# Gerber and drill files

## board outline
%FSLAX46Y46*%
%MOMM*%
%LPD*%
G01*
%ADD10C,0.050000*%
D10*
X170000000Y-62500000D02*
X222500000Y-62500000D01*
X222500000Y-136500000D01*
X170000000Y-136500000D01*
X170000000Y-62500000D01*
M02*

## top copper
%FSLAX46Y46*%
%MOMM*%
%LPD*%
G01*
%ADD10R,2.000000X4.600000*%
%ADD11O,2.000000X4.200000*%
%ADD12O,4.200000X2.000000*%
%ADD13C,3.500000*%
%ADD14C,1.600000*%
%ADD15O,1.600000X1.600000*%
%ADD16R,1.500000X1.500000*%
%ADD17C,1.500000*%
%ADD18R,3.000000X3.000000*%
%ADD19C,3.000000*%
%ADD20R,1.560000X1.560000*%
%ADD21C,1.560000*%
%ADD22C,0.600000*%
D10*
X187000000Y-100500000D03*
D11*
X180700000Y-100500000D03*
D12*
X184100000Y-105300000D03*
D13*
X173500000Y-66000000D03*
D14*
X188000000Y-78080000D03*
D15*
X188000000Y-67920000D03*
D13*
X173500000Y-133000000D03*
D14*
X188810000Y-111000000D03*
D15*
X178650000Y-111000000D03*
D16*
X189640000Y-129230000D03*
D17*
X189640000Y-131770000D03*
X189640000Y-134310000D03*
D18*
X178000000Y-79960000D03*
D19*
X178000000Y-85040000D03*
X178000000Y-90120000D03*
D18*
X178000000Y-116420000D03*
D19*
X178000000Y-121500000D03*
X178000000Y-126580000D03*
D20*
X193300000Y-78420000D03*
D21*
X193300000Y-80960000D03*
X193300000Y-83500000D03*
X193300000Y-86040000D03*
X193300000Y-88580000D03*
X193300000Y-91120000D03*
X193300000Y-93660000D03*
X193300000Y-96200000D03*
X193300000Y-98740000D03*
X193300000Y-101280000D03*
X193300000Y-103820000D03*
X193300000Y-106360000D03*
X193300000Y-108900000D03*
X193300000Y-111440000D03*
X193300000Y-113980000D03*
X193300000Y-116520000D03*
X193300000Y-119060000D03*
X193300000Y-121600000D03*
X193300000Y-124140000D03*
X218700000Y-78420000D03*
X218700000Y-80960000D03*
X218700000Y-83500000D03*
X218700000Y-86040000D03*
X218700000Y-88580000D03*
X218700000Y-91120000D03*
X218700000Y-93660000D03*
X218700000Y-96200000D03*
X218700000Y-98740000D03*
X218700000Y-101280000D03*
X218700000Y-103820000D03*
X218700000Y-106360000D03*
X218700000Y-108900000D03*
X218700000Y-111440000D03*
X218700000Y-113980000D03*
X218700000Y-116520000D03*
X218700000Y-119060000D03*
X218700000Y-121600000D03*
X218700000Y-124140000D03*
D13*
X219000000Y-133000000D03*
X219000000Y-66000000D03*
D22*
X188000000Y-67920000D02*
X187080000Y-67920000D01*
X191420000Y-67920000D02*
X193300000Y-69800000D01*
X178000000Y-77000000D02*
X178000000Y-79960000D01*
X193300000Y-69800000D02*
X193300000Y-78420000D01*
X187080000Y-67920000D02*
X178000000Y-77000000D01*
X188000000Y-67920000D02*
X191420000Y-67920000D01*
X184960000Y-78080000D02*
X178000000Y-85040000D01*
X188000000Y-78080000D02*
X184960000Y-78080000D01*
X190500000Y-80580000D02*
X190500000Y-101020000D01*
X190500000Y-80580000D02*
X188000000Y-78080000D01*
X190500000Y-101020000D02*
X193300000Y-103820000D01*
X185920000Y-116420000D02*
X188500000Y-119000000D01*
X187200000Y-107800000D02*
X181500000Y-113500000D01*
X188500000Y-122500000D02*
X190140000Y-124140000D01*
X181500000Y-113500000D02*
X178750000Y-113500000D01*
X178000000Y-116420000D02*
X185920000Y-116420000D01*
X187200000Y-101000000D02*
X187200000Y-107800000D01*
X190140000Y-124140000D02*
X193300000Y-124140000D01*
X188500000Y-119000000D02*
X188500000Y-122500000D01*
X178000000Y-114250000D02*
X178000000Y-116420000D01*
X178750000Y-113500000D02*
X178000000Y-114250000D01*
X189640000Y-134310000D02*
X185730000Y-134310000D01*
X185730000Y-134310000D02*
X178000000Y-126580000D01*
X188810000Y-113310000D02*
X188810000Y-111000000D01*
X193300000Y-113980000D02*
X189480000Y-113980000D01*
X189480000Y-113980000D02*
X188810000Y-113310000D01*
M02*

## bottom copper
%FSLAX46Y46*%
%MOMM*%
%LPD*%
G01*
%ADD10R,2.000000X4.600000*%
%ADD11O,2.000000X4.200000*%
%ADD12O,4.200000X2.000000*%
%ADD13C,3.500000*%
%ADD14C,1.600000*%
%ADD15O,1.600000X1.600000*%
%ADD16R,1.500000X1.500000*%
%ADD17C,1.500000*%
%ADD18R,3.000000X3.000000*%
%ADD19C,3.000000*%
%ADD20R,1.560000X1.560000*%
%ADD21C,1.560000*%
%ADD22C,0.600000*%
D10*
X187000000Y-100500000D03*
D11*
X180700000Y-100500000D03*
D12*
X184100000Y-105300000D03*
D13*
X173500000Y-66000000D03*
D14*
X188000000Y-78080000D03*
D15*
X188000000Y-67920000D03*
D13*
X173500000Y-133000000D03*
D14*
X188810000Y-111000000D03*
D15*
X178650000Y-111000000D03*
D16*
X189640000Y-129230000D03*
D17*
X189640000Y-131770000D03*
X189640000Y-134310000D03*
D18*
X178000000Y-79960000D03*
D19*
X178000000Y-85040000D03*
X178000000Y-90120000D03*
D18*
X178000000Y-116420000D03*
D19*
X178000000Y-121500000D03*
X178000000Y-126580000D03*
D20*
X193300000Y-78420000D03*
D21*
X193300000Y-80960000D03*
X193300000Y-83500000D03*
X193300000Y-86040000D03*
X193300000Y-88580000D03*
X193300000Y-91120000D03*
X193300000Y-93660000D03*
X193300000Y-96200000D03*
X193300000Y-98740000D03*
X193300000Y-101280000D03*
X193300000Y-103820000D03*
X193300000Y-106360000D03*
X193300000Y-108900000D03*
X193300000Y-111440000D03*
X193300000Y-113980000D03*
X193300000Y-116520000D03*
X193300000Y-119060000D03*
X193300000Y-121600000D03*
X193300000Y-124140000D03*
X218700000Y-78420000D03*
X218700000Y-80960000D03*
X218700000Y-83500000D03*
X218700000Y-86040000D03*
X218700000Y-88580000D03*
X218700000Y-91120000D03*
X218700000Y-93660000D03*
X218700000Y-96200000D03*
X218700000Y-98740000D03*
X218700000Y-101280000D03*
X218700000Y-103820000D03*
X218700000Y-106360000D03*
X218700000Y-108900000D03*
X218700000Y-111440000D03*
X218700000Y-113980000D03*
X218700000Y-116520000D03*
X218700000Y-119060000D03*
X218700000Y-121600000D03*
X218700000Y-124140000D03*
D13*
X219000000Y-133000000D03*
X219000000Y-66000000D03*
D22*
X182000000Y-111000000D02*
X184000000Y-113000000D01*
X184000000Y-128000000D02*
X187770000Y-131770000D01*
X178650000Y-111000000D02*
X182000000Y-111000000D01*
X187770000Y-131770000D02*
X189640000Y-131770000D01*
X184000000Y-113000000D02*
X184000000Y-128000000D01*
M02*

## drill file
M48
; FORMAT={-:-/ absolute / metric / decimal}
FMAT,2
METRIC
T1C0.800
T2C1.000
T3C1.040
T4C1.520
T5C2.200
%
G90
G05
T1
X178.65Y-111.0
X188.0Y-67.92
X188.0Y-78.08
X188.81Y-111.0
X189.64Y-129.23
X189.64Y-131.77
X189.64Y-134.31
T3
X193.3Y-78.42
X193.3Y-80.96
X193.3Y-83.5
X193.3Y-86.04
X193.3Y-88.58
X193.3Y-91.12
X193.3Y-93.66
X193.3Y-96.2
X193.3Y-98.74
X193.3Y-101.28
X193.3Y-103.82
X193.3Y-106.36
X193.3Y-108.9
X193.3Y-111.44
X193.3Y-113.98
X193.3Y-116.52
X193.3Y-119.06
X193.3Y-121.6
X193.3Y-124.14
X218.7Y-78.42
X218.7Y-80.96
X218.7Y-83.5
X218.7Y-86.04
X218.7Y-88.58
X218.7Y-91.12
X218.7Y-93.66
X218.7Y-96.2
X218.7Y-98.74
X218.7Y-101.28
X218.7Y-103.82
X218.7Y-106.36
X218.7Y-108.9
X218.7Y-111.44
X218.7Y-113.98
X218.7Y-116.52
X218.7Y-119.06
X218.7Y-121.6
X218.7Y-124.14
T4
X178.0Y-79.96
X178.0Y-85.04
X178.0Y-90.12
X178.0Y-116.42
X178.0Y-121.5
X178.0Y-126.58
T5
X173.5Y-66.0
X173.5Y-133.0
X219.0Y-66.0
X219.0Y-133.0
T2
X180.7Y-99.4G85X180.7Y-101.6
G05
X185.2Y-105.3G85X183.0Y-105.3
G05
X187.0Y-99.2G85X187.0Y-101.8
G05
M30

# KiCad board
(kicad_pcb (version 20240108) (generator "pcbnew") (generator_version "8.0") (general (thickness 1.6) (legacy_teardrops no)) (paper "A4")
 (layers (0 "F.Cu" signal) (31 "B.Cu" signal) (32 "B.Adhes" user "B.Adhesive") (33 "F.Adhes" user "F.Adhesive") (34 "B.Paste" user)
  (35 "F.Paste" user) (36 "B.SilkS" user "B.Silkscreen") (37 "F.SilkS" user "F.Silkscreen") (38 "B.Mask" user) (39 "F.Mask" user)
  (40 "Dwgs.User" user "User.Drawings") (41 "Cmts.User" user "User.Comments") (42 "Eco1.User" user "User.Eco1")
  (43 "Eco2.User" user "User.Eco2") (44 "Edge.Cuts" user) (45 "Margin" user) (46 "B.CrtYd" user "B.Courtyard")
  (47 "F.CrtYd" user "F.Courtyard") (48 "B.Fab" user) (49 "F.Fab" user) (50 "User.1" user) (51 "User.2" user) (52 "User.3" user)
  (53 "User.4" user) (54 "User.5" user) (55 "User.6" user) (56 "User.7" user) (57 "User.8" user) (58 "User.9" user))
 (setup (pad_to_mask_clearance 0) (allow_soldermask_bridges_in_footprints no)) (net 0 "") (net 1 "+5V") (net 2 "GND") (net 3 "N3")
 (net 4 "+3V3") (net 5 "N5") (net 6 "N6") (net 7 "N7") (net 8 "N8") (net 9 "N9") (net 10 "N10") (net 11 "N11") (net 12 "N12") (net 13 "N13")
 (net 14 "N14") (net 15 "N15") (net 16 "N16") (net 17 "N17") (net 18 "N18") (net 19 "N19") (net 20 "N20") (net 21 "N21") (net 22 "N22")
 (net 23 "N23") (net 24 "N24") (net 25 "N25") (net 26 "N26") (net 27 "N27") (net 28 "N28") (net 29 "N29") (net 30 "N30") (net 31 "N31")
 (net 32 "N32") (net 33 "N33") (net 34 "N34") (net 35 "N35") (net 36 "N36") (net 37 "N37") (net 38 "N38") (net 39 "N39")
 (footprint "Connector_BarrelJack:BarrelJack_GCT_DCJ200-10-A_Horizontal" (layer "F.Cu") (at 187 100.5 -90)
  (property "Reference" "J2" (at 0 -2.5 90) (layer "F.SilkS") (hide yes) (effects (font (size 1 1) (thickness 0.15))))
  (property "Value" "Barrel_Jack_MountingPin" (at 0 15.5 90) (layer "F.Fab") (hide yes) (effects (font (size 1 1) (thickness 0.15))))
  (pad "1" thru_hole rect (at 0 0 270) (size 4.6 2) (drill oval 3.6 1) (layers "*.Cu" "*.Mask") (remove_unused_layers no) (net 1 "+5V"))
  (pad "2" thru_hole oval (at 0 6.3 270) (size 4.2 2) (drill oval 3.2 1) (layers "*.Cu" "*.Mask") (remove_unused_layers no) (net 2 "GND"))
  (pad "3" thru_hole oval (at 4.8 2.9 270) (size 2 4.2) (drill oval 1 3.2) (layers "*.Cu" "*.Mask") (remove_unused_layers no)))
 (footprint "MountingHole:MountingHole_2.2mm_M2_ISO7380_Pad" (layer "F.Cu") (at 173.5 66)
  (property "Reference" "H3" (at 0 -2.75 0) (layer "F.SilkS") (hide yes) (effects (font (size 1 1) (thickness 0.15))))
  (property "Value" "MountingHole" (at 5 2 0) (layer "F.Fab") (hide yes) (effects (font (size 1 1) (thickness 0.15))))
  (pad "1" thru_hole circle (at 0 0) (size 3.5 3.5) (drill 2.2) (layers "*.Cu" "*.Mask") (remove_unused_layers no)))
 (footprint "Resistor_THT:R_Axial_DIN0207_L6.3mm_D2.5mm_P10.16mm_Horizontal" (layer "F.Cu") (at 188 78.08 90)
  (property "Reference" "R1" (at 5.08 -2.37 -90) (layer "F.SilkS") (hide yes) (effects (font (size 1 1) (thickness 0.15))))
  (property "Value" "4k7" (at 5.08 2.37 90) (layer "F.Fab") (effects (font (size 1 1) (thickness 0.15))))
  (pad "1" thru_hole circle (at 0 0 90) (size 1.6 1.6) (drill 0.8) (layers "*.Cu" "*.Mask") (remove_unused_layers no) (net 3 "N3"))
  (pad "2" thru_hole oval (at 10.16 0 90) (size 1.6 1.6) (drill 0.8) (layers "*.Cu" "*.Mask") (remove_unused_layers no) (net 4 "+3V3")))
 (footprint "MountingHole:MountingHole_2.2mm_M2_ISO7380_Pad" (layer "F.Cu") (at 173.5 133)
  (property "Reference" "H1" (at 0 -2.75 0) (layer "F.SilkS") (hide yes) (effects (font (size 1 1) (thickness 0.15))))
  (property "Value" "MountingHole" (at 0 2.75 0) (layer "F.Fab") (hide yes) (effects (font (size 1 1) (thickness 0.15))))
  (pad "1" thru_hole circle (at 0 0) (size 3.5 3.5) (drill 2.2) (layers "*.Cu" "*.Mask") (remove_unused_layers no)))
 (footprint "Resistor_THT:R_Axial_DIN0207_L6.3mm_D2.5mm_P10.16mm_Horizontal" (layer "F.Cu") (at 188.81 111 180)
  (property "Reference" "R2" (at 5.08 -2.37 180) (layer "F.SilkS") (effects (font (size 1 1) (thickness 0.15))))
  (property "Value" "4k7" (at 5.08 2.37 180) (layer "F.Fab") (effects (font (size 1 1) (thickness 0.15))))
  (pad "1" thru_hole circle (at 0 0 180) (size 1.6 1.6) (drill 0.8) (layers "*.Cu" "*.Mask") (remove_unused_layers no) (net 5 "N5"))
  (pad "2" thru_hole oval (at 10.16 0 180) (size 1.6 1.6) (drill 0.8) (layers "*.Cu" "*.Mask") (remove_unused_layers no) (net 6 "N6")))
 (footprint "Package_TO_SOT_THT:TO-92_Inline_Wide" (layer "F.Cu") (at 189.64 129.23 -90)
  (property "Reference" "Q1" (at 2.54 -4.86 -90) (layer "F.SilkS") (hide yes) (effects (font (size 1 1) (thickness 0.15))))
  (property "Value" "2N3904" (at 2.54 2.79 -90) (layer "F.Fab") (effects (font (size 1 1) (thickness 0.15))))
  (pad "1" thru_hole rect (at 0 0 270) (size 1.5 1.5) (drill 0.8) (layers "*.Cu" "*.Mask") (remove_unused_layers no) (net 2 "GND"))
  (pad "2" thru_hole circle (at 2.54 0 270) (size 1.5 1.5) (drill 0.8) (layers "*.Cu" "*.Mask") (remove_unused_layers no) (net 6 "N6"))
  (pad "3" thru_hole circle (at 5.08 0 270) (size 1.5 1.5) (drill 0.8) (layers "*.Cu" "*.Mask") (remove_unused_layers no) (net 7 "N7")))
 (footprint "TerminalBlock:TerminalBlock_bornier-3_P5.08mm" (layer "F.Cu") (at 178 79.96 -90)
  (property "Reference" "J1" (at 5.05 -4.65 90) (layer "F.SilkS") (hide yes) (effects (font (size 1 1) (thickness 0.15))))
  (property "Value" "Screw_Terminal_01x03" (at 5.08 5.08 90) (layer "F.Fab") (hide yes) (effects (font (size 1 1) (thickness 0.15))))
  (pad "1" thru_hole rect (at 0 0 270) (size 3 3) (drill 1.52) (layers "*.Cu" "*.Mask") (remove_unused_layers no) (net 4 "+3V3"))
  (pad "2" thru_hole circle (at 5.08 0 270) (size 3 3) (drill 1.52) (layers "*.Cu" "*.Mask") (remove_unused_layers no) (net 3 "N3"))
  (pad "3" thru_hole circle (at 10.16 0 270) (size 3 3) (drill 1.52) (layers "*.Cu" "*.Mask") (remove_unused_layers no) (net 2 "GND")))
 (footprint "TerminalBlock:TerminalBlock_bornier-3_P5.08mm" (layer "F.Cu") (at 178 116.42 -90)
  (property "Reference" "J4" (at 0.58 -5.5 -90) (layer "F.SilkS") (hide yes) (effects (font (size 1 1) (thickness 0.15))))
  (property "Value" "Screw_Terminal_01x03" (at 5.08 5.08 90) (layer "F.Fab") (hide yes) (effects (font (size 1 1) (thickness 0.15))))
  (pad "1" thru_hole rect (at 0 0 270) (size 3 3) (drill 1.52) (layers "*.Cu" "*.Mask") (remove_unused_layers no) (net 1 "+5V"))
  (pad "2" thru_hole circle (at 5.08 0 270) (size 3 3) (drill 1.52) (layers "*.Cu" "*.Mask") (remove_unused_layers no) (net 2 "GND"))
  (pad "3" thru_hole circle (at 10.16 0 270) (size 3 3) (drill 1.52) (layers "*.Cu" "*.Mask") (remove_unused_layers no) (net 7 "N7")))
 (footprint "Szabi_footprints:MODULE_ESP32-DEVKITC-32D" (layer "F.Cu") (at 206 98.18)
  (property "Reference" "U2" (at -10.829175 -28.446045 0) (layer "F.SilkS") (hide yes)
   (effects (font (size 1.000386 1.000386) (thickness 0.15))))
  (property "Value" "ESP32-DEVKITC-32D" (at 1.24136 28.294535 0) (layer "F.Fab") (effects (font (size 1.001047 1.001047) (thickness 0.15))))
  (pad "J2-1" thru_hole rect (at -12.7 -19.76) (size 1.56 1.56) (drill 1.04) (layers "*.Cu" "*.Mask") (remove_unused_layers no)
   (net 4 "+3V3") (solder_mask_margin 0.102))
  (pad "J2-2" thru_hole circle (at -12.7 -17.22) (size 1.56 1.56) (drill 1.04) (layers "*.Cu" "*.Mask") (remove_unused_layers no)
   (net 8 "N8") (solder_mask_margin 0.102))
  (pad "J2-3" thru_hole circle (at -12.7 -14.68) (size 1.56 1.56) (drill 1.04) (layers "*.Cu" "*.Mask") (remove_unused_layers no)
   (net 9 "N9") (solder_mask_margin 0.102))
  (pad "J2-4" thru_hole circle (at -12.7 -12.14) (size 1.56 1.56) (drill 1.04) (layers "*.Cu" "*.Mask") (remove_unused_layers no)
   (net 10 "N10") (solder_mask_margin 0.102))
  (pad "J2-5" thru_hole circle (at -12.7 -9.6) (size 1.56 1.56) (drill 1.04) (layers "*.Cu" "*.Mask") (remove_unused_layers no)
   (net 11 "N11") (solder_mask_margin 0.102))
  (pad "J2-6" thru_hole circle (at -12.7 -7.06) (size 1.56 1.56) (drill 1.04) (layers "*.Cu" "*.Mask") (remove_unused_layers no)
   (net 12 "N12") (solder_mask_margin 0.102))
  (pad "J2-7" thru_hole circle (at -12.7 -4.52) (size 1.56 1.56) (drill 1.04) (layers "*.Cu" "*.Mask") (remove_unused_layers no)
   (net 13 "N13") (solder_mask_margin 0.102))
  (pad "J2-8" thru_hole circle (at -12.7 -1.98) (size 1.56 1.56) (drill 1.04) (layers "*.Cu" "*.Mask") (remove_unused_layers no)
   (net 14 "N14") (solder_mask_margin 0.102))
  (pad "J2-9" thru_hole circle (at -12.7 0.56) (size 1.56 1.56) (drill 1.04) (layers "*.Cu" "*.Mask") (remove_unused_layers no)
   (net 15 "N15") (solder_mask_margin 0.102))
  (pad "J2-10" thru_hole circle (at -12.7 3.1) (size 1.56 1.56) (drill 1.04) (layers "*.Cu" "*.Mask") (remove_unused_layers no)
   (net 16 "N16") (solder_mask_margin 0.102))
  (pad "J2-11" thru_hole circle (at -12.7 5.64) (size 1.56 1.56) (drill 1.04) (layers "*.Cu" "*.Mask") (remove_unused_layers no)
   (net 3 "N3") (solder_mask_margin 0.102))
  (pad "J2-12" thru_hole circle (at -12.7 8.18) (size 1.56 1.56) (drill 1.04) (layers "*.Cu" "*.Mask") (remove_unused_layers no)
   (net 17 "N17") (solder_mask_margin 0.102))
  (pad "J2-13" thru_hole circle (at -12.7 10.72) (size 1.56 1.56) (drill 1.04) (layers "*.Cu" "*.Mask") (remove_unused_layers no)
   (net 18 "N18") (solder_mask_margin 0.102))
  (pad "J2-14" thru_hole circle (at -12.7 13.26) (size 1.56 1.56) (drill 1.04) (layers "*.Cu" "*.Mask") (remove_unused_layers no)
   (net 2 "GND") (solder_mask_margin 0.102))
  (pad "J2-15" thru_hole circle (at -12.7 15.8) (size 1.56 1.56) (drill 1.04) (layers "*.Cu" "*.Mask") (remove_unused_layers no)
   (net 5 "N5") (solder_mask_margin 0.102))
  (pad "J2-16" thru_hole circle (at -12.7 18.34) (size 1.56 1.56) (drill 1.04) (layers "*.Cu" "*.Mask") (remove_unused_layers no)
   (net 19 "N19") (solder_mask_margin 0.102))
  (pad "J2-17" thru_hole circle (at -12.7 20.88) (size 1.56 1.56) (drill 1.04) (layers "*.Cu" "*.Mask") (remove_unused_layers no)
   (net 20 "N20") (solder_mask_margin 0.102))
  (pad "J2-18" thru_hole circle (at -12.7 23.42) (size 1.56 1.56) (drill 1.04) (layers "*.Cu" "*.Mask") (remove_unused_layers no)
   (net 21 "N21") (solder_mask_margin 0.102))
  (pad "J2-19" thru_hole circle (at -12.7 25.96) (size 1.56 1.56) (drill 1.04) (layers "*.Cu" "*.Mask") (remove_unused_layers no)
   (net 1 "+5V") (solder_mask_margin 0.102))
  (pad "J3-1" thru_hole circle (at 12.7 -19.76) (size 1.56 1.56) (drill 1.04) (layers "*.Cu" "*.Mask") (remove_unused_layers no)
   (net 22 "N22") (solder_mask_margin 0.102))
  (pad "J3-2" thru_hole circle (at 12.7 -17.22) (size 1.56 1.56) (drill 1.04) (layers "*.Cu" "*.Mask") (remove_unused_layers no)
   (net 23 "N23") (solder_mask_margin 0.102))
  (pad "J3-3" thru_hole circle (at 12.7 -14.68) (size 1.56 1.56) (drill 1.04) (layers "*.Cu" "*.Mask") (remove_unused_layers no)
   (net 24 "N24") (solder_mask_margin 0.102))
  (pad "J3-4" thru_hole circle (at 12.7 -12.14) (size 1.56 1.56) (drill 1.04) (layers "*.Cu" "*.Mask") (remove_unused_layers no)
   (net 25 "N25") (solder_mask_margin 0.102))
  (pad "J3-5" thru_hole circle (at 12.7 -9.6) (size 1.56 1.56) (drill 1.04) (layers "*.Cu" "*.Mask") (remove_unused_layers no)
   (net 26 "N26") (solder_mask_margin 0.102))
  (pad "J3-6" thru_hole circle (at 12.7 -7.06) (size 1.56 1.56) (drill 1.04) (layers "*.Cu" "*.Mask") (remove_unused_layers no)
   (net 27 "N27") (solder_mask_margin 0.102))
  (pad "J3-7" thru_hole circle (at 12.7 -4.52) (size 1.56 1.56) (drill 1.04) (layers "*.Cu" "*.Mask") (remove_unused_layers no)
   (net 2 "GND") (solder_mask_margin 0.102))
  (pad "J3-8" thru_hole circle (at 12.7 -1.98) (size 1.56 1.56) (drill 1.04) (layers "*.Cu" "*.Mask") (remove_unused_layers no)
   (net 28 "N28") (solder_mask_margin 0.102))
  (pad "J3-9" thru_hole circle (at 12.7 0.56) (size 1.56 1.56) (drill 1.04) (layers "*.Cu" "*.Mask") (remove_unused_layers no)
   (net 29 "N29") (solder_mask_margin 0.102))
  (pad "J3-10" thru_hole circle (at 12.7 3.1) (size 1.56 1.56) (drill 1.04) (layers "*.Cu" "*.Mask") (remove_unused_layers no)
   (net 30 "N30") (solder_mask_margin 0.102))
  (pad "J3-11" thru_hole circle (at 12.7 5.64) (size 1.56 1.56) (drill 1.04) (layers "*.Cu" "*.Mask") (remove_unused_layers no)
   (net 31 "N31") (solder_mask_margin 0.102))
  (pad "J3-12" thru_hole circle (at 12.7 8.18) (size 1.56 1.56) (drill 1.04) (layers "*.Cu" "*.Mask") (remove_unused_layers no)
   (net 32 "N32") (solder_mask_margin 0.102))
  (pad "J3-13" thru_hole circle (at 12.7 10.72) (size 1.56 1.56) (drill 1.04) (layers "*.Cu" "*.Mask") (remove_unused_layers no)
   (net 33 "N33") (solder_mask_margin 0.102))
  (pad "J3-14" thru_hole circle (at 12.7 13.26) (size 1.56 1.56) (drill 1.04) (layers "*.Cu" "*.Mask") (remove_unused_layers no)
   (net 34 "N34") (solder_mask_margin 0.102))
  (pad "J3-15" thru_hole circle (at 12.7 15.8) (size 1.56 1.56) (drill 1.04) (layers "*.Cu" "*.Mask") (remove_unused_layers no)
   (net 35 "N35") (solder_mask_margin 0.102))
  (pad "J3-16" thru_hole circle (at 12.7 18.34) (size 1.56 1.56) (drill 1.04) (layers "*.Cu" "*.Mask") (remove_unused_layers no)
   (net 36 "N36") (solder_mask_margin 0.102))
  (pad "J3-17" thru_hole circle (at 12.7 20.88) (size 1.56 1.56) (drill 1.04) (layers "*.Cu" "*.Mask") (remove_unused_layers no)
   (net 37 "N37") (solder_mask_margin 0.102))
  (pad "J3-18" thru_hole circle (at 12.7 23.42) (size 1.56 1.56) (drill 1.04) (layers "*.Cu" "*.Mask") (remove_unused_layers no)
   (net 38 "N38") (solder_mask_margin 0.102))
  (pad "J3-19" thru_hole circle (at 12.7 25.96) (size 1.56 1.56) (drill 1.04) (layers "*.Cu" "*.Mask") (remove_unused_layers no)
   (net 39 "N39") (solder_mask_margin 0.102)))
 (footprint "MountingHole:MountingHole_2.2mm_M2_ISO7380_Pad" (layer "F.Cu") (at 219 133)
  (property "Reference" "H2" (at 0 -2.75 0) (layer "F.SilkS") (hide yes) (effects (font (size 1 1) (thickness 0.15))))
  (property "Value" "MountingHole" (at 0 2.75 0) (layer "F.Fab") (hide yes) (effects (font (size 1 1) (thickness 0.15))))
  (pad "1" thru_hole circle (at 0 0) (size 3.5 3.5) (drill 2.2) (layers "*.Cu" "*.Mask") (remove_unused_layers no)))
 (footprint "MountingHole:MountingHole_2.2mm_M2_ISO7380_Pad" (layer "F.Cu") (at 219 66)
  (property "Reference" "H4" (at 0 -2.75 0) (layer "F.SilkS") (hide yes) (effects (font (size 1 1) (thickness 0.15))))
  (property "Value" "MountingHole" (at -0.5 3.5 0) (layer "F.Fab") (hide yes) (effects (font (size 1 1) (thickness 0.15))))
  (pad "1" thru_hole circle (at 0 0) (size 3.5 3.5) (drill 2.2) (layers "*.Cu" "*.Mask") (remove_unused_layers no)))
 (gr_rect (start 170 62.5) (end 222.5 136.5) (stroke (width 0.05) (type solid)) (fill none) (layer "Edge.Cuts"))
 (segment (start 188 67.92) (end 187.08 67.92) (width 0.6) (layer "F.Cu") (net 4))
 (segment (start 191.42 67.92) (end 193.3 69.8) (width 0.6) (layer "F.Cu") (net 4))
 (segment (start 178 77) (end 178 79.96) (width 0.6) (layer "F.Cu") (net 4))
 (segment (start 193.3 69.8) (end 193.3 78.42) (width 0.6) (layer "F.Cu") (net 4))
 (segment (start 187.08 67.92) (end 178 77) (width 0.6) (layer "F.Cu") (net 4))
 (segment (start 188 67.92) (end 191.42 67.92) (width 0.6) (layer "F.Cu") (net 4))
 (segment (start 184.96 78.08) (end 178 85.04) (width 0.6) (layer "F.Cu") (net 3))
 (segment (start 188 78.08) (end 184.96 78.08) (width 0.6) (layer "F.Cu") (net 3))
 (segment (start 190.5 80.58) (end 190.5 101.02) (width 0.6) (layer "F.Cu") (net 3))
 (segment (start 190.5 80.58) (end 188 78.08) (width 0.6) (layer "F.Cu") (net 3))
 (segment (start 190.5 101.02) (end 193.3 103.82) (width 0.6) (layer "F.Cu") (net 3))
 (segment (start 185.92 116.42) (end 188.5 119) (width 0.6) (layer "F.Cu") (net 1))
 (segment (start 187.2 107.8) (end 181.5 113.5) (width 0.6) (layer "F.Cu") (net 1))
 (segment (start 188.5 122.5) (end 190.14 124.14) (width 0.6) (layer "F.Cu") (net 1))
 (segment (start 181.5 113.5) (end 178.75 113.5) (width 0.6) (layer "F.Cu") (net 1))
 (segment (start 178 116.42) (end 185.92 116.42) (width 0.6) (layer "F.Cu") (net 1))
 (segment (start 187.2 101) (end 187.2 107.8) (width 0.6) (layer "F.Cu") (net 1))
 (segment (start 190.14 124.14) (end 193.3 124.14) (width 0.6) (layer "F.Cu") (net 1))
 (segment (start 188.5 119) (end 188.5 122.5) (width 0.6) (layer "F.Cu") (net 1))
 (segment (start 178 114.25) (end 178 116.42) (width 0.6) (layer "F.Cu") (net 1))
 (segment (start 178.75 113.5) (end 178 114.25) (width 0.6) (layer "F.Cu") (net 1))
 (segment (start 182 111) (end 184 113) (width 0.6) (layer "B.Cu") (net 6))
 (segment (start 184 128) (end 187.77 131.77) (width 0.6) (layer "B.Cu") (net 6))
 (segment (start 178.65 111) (end 182 111) (width 0.6) (layer "B.Cu") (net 6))
 (segment (start 187.77 131.77) (end 189.64 131.77) (width 0.6) (layer "B.Cu") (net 6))
 (segment (start 184 113) (end 184 128) (width 0.6) (layer "B.Cu") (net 6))
 (segment (start 189.64 134.31) (end 185.73 134.31) (width 0.6) (layer "F.Cu") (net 7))
 (segment (start 185.73 134.31) (end 178 126.58) (width 0.6) (layer "F.Cu") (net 7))
 (segment (start 188.81 113.31) (end 188.81 111) (width 0.6) (layer "F.Cu") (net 5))
 (segment (start 193.3 113.98) (end 189.48 113.98) (width 0.6) (layer "F.Cu") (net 5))
 (segment (start 189.48 113.98) (end 188.81 113.31) (width 0.6) (layer "F.Cu") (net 5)))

